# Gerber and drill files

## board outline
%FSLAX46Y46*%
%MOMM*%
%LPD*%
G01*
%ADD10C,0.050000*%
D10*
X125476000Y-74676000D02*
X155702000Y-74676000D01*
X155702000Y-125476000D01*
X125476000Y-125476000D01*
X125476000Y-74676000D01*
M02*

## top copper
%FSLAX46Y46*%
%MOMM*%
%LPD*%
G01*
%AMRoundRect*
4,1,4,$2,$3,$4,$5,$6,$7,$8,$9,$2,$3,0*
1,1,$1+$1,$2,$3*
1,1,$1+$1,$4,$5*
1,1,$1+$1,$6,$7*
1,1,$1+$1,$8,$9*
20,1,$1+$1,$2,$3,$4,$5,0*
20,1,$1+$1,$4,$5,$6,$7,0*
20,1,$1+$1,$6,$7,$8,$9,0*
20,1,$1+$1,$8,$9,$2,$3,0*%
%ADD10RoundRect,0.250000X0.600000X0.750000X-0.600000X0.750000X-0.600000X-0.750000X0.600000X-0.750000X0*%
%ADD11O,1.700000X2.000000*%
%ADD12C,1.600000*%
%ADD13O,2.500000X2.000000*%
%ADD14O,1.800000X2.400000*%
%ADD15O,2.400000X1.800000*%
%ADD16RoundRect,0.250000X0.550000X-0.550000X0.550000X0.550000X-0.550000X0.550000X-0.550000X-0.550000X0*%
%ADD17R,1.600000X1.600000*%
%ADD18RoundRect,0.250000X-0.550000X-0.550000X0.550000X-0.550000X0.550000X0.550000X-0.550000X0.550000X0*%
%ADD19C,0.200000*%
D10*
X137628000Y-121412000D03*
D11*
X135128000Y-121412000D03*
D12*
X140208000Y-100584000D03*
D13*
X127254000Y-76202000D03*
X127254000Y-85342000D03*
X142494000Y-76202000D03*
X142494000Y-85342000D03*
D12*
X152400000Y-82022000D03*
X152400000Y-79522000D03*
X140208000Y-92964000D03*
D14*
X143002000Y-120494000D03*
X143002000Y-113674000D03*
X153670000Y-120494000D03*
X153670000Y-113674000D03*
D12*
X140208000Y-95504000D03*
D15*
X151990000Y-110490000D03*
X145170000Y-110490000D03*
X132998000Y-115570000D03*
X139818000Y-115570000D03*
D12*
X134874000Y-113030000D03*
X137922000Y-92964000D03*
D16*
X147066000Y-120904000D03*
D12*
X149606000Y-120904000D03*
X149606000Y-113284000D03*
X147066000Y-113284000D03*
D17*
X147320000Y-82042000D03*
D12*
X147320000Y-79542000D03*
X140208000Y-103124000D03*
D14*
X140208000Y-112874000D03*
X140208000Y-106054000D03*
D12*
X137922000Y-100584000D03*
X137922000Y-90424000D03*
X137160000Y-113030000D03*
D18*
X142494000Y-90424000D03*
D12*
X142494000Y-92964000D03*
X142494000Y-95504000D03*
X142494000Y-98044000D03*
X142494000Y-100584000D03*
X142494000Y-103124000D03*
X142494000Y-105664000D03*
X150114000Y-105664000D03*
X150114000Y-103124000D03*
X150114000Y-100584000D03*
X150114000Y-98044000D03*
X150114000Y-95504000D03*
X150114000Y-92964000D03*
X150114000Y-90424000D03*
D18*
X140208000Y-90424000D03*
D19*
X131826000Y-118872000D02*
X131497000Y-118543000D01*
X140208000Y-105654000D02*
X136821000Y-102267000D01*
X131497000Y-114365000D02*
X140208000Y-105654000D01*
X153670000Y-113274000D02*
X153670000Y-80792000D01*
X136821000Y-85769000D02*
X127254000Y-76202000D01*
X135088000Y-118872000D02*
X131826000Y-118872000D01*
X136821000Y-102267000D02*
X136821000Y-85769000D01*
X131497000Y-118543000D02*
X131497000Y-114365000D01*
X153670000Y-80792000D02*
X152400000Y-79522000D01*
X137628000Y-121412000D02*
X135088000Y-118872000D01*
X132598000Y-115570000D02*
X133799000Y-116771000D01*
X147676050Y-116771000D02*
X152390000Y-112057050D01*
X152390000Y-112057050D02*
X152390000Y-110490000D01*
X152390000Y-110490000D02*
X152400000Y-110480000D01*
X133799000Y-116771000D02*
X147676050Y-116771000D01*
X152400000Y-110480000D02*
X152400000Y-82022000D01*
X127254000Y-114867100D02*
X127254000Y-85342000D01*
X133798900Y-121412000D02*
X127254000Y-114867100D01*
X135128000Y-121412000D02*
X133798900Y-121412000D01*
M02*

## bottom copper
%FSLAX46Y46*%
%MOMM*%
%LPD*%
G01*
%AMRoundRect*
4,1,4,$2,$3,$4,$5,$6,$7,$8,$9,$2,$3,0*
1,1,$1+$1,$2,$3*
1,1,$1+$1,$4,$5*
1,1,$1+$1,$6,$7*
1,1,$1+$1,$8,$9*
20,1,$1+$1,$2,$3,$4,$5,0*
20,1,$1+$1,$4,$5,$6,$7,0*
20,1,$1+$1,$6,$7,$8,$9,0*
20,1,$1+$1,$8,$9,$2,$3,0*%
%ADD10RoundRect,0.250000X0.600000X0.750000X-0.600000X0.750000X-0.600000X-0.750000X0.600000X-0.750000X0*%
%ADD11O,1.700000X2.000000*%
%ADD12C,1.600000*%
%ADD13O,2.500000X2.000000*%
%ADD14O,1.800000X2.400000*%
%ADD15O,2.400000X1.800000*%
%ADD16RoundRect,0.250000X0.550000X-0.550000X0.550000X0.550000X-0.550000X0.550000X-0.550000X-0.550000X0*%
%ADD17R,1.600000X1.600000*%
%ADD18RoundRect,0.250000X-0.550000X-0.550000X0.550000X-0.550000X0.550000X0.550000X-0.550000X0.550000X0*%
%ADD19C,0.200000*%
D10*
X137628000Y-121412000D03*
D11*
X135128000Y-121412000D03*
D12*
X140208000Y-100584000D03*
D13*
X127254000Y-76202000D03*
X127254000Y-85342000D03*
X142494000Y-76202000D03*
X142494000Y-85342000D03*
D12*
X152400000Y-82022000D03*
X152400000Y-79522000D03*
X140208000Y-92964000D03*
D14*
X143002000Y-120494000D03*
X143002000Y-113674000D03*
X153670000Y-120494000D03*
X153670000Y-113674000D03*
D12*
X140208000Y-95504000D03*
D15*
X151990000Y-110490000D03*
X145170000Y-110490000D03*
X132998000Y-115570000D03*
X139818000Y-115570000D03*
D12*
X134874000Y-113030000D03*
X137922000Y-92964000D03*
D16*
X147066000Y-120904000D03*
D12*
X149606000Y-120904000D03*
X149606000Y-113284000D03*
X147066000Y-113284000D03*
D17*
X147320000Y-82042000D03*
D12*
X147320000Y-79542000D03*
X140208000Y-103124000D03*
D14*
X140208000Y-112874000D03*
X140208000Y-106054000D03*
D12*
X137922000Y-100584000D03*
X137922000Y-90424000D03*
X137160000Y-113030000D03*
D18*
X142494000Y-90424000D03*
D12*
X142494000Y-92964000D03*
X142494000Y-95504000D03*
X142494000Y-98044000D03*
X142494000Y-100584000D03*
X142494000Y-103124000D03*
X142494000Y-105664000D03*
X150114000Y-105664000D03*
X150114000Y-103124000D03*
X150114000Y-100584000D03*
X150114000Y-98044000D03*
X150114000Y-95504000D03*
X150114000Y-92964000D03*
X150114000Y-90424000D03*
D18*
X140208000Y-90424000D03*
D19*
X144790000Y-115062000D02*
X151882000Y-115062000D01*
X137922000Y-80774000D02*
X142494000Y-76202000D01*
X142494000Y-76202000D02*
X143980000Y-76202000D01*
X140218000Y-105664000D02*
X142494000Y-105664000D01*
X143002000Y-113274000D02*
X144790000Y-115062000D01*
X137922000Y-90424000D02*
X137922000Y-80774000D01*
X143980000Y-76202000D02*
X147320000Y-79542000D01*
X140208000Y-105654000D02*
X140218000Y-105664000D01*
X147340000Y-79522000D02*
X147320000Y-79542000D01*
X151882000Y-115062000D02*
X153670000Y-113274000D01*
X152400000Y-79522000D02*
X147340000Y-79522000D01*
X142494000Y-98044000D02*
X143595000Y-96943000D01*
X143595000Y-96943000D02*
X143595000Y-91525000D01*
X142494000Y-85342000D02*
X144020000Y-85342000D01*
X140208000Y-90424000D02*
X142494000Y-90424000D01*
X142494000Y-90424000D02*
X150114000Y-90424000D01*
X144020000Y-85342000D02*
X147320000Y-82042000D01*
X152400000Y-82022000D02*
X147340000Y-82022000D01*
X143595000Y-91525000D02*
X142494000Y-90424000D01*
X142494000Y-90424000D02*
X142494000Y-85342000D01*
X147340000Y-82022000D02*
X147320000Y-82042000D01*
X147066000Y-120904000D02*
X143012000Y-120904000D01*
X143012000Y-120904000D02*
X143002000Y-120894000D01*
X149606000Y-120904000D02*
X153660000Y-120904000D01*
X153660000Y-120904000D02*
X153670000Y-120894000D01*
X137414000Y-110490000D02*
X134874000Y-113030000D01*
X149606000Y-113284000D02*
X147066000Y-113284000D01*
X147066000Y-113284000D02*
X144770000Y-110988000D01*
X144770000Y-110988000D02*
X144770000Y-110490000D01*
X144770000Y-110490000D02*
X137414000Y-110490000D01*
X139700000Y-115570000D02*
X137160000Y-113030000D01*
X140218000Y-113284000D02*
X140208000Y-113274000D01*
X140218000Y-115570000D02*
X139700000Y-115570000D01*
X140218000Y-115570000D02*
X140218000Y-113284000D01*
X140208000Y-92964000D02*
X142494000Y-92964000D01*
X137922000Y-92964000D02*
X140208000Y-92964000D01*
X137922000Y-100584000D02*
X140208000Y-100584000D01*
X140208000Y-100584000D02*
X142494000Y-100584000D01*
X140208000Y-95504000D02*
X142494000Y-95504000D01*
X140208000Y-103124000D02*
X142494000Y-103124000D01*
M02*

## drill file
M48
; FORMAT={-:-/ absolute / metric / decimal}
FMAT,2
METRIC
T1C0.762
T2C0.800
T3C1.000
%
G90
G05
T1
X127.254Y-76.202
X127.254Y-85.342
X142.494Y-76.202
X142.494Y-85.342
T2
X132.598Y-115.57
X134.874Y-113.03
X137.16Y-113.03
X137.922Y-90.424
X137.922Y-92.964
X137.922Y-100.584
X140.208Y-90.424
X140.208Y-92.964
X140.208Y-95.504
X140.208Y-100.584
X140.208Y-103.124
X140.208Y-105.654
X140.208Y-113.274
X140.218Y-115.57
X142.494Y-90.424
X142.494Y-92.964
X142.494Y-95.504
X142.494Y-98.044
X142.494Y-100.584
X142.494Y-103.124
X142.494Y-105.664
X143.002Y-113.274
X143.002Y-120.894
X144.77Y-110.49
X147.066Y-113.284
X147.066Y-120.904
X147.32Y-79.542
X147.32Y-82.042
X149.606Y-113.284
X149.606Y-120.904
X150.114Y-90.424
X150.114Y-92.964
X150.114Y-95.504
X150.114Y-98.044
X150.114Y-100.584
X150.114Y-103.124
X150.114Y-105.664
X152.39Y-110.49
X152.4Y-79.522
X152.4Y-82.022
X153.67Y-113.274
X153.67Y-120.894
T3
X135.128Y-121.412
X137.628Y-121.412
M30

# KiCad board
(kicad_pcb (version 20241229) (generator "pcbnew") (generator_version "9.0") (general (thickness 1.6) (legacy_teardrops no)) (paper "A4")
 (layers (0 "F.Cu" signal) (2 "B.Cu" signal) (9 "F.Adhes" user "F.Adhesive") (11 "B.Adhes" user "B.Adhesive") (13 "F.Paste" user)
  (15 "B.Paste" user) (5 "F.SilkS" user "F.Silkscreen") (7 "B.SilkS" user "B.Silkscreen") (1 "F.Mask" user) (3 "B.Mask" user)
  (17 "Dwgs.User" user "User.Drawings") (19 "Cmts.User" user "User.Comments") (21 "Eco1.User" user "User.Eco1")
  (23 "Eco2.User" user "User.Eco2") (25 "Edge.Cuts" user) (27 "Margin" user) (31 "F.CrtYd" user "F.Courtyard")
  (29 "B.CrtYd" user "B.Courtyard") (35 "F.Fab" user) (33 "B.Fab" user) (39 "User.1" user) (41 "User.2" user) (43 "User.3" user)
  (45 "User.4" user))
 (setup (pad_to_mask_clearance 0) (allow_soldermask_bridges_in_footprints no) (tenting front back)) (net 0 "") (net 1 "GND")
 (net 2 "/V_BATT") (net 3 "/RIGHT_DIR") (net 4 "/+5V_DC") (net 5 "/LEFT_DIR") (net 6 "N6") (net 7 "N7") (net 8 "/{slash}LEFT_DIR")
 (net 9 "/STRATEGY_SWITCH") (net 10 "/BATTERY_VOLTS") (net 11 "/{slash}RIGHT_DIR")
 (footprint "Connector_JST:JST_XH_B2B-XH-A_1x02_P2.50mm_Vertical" (layer "F.Cu") (at 137.628 121.412 180)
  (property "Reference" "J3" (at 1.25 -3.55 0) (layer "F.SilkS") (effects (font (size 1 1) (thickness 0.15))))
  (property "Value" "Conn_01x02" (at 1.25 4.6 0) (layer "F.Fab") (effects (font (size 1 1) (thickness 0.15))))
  (pad "1" thru_hole roundrect (at 0 0 180) (size 1.7 2) (drill 1) (layers "*.Cu" "*.Mask") (remove_unused_layers no)
   (roundrect_rratio 0.147059) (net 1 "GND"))
  (pad "2" thru_hole oval (at 2.5 0 180) (size 1.7 2) (drill 1) (layers "*.Cu" "*.Mask") (remove_unused_layers no) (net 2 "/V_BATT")))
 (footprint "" (layer "F.Cu") (at 140.208 100.584)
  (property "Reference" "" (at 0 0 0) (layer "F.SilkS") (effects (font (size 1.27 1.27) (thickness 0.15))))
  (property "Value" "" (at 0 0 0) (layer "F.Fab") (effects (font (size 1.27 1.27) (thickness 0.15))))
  (pad "5" thru_hole circle (at 0 0) (size 1.6 1.6) (drill 0.8) (layers "*.Cu" "*.Mask") (remove_unused_layers no) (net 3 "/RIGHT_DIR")))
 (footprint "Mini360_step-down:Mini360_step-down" (layer "F.Cu") (at 134.874 80.772)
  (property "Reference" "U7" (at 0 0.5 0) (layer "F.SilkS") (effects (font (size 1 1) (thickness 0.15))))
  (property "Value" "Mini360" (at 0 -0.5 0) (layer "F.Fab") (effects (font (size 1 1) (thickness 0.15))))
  (pad "1" thru_hole oval (at -7.62 -4.57) (size 2.5 2) (drill 0.762) (layers "*.Cu" "*.Mask") (remove_unused_layers no) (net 1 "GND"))
  (pad "2" thru_hole oval (at -7.62 4.57) (size 2.5 2) (drill 0.762) (layers "*.Cu" "*.Mask") (remove_unused_layers no) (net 2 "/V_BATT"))
  (pad "3" thru_hole oval (at 7.62 -4.57) (size 2.5 2) (drill 0.762) (layers "*.Cu" "*.Mask") (remove_unused_layers no) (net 1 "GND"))
  (pad "4" thru_hole oval (at 7.62 4.57) (size 2.5 2) (drill 0.762) (layers "*.Cu" "*.Mask") (remove_unused_layers no) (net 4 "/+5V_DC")))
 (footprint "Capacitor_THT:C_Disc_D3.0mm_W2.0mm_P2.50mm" (layer "F.Cu") (at 152.4 82.022 90)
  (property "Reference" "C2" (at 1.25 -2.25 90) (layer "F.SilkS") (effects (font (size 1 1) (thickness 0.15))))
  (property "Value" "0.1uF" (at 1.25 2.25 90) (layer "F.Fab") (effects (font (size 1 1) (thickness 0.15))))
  (pad "1" thru_hole circle (at 0 0 90) (size 1.6 1.6) (drill 0.8) (layers "*.Cu" "*.Mask") (remove_unused_layers no) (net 4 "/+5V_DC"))
  (pad "2" thru_hole circle (at 2.5 0 90) (size 1.6 1.6) (drill 0.8) (layers "*.Cu" "*.Mask") (remove_unused_layers no) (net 1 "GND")))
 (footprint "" (layer "F.Cu") (at 140.208 92.964)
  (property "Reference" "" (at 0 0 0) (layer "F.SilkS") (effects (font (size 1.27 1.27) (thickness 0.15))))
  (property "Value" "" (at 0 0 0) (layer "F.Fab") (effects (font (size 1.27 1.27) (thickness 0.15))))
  (pad "2" thru_hole circle (at 0 0) (size 1.6 1.6) (drill 0.8) (layers "*.Cu" "*.Mask") (remove_unused_layers no) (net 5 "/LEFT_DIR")))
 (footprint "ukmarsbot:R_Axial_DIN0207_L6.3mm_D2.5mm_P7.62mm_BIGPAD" (layer "F.Cu") (at 143.002 120.894 90)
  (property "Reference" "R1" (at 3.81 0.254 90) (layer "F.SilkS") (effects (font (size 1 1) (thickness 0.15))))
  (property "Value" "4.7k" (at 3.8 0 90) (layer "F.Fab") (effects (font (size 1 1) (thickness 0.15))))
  (pad "1" thru_hole oval (at 0 0 90) (size 2.4 1.8) (drill 0.8 (offset 0.4 0)) (layers "*.Cu" "*.Mask") (remove_unused_layers no)
   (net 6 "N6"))
  (pad "2" thru_hole oval (at 7.62 0 90) (size 2.4 1.8) (drill 0.8 (offset -0.4 0)) (layers "*.Cu" "*.Mask") (remove_unused_layers no)
   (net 1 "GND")))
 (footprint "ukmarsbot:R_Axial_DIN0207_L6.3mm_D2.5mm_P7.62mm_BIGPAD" (layer "F.Cu") (at 153.67 120.894 90)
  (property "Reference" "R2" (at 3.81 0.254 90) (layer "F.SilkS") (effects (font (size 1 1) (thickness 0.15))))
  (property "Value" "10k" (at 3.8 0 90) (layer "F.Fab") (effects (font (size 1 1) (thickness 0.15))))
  (pad "1" thru_hole oval (at 0 0 90) (size 2.4 1.8) (drill 0.8 (offset 0.4 0)) (layers "*.Cu" "*.Mask") (remove_unused_layers no)
   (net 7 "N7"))
  (pad "2" thru_hole oval (at 7.62 0 90) (size 2.4 1.8) (drill 0.8 (offset -0.4 0)) (layers "*.Cu" "*.Mask") (remove_unused_layers no)
   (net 1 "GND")))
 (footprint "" (layer "F.Cu") (at 140.208 95.504)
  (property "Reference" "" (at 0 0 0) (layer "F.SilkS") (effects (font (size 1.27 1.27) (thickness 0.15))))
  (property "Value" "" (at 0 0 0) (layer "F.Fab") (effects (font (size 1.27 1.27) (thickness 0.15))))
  (pad "3" thru_hole circle (at 0 0) (size 1.6 1.6) (drill 0.8) (layers "*.Cu" "*.Mask") (remove_unused_layers no)
   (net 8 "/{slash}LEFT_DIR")))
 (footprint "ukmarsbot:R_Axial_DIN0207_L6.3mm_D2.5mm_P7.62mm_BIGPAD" (layer "F.Cu") (at 152.39 110.49 180)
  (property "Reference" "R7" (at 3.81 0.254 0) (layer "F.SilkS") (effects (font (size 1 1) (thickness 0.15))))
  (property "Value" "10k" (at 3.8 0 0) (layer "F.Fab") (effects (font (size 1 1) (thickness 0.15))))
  (pad "1" thru_hole oval (at 0 0 180) (size 2.4 1.8) (drill 0.8 (offset 0.4 0)) (layers "*.Cu" "*.Mask") (remove_unused_layers no)
   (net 4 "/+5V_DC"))
  (pad "2" thru_hole oval (at 7.62 0 180) (size 2.4 1.8) (drill 0.8 (offset -0.4 0)) (layers "*.Cu" "*.Mask") (remove_unused_layers no)
   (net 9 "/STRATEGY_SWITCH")))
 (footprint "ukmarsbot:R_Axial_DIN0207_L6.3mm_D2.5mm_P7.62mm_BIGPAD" (layer "F.Cu") (at 132.598 115.57)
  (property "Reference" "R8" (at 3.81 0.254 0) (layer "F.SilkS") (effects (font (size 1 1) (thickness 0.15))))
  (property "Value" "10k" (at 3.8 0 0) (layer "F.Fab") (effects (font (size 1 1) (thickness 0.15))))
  (pad "1" thru_hole oval (at 0 0) (size 2.4 1.8) (drill 0.8 (offset 0.4 0)) (layers "*.Cu" "*.Mask") (remove_unused_layers no)
   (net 4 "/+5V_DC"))
  (pad "2" thru_hole oval (at 7.62 0) (size 2.4 1.8) (drill 0.8 (offset -0.4 0)) (layers "*.Cu" "*.Mask") (remove_unused_layers no)
   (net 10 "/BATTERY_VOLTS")))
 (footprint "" (layer "F.Cu") (at 134.874 113.03)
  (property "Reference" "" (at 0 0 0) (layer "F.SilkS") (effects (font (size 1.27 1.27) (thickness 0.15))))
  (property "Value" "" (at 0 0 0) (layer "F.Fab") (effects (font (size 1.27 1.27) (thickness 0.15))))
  (pad "5" thru_hole circle (at 0 0) (size 1.6 1.6) (drill 0.8) (layers "*.Cu" "*.Mask") (remove_unused_layers no)
   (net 9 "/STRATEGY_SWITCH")))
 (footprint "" (layer "F.Cu") (at 137.922 92.964)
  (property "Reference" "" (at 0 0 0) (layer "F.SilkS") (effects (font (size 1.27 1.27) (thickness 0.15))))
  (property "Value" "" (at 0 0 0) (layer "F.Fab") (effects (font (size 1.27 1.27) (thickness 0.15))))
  (pad "2" thru_hole circle (at 0 0) (size 1.6 1.6) (drill 0.8) (layers "*.Cu" "*.Mask") (remove_unused_layers no) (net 5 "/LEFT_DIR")))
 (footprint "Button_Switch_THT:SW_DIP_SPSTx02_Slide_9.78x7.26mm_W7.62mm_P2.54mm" (layer "F.Cu") (at 147.066 120.904 90)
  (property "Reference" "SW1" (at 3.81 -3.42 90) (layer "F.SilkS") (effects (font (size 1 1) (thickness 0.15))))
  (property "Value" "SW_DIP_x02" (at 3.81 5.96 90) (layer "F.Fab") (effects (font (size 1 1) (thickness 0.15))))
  (pad "1" thru_hole roundrect (at 0 0 90) (size 1.6 1.6) (drill 0.8) (layers "*.Cu" "*.Mask") (remove_unused_layers no)
   (roundrect_rratio 0.15625) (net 6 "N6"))
  (pad "2" thru_hole circle (at 0 2.54 90) (size 1.6 1.6) (drill 0.8) (layers "*.Cu" "*.Mask") (remove_unused_layers no) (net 7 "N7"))
  (pad "3" thru_hole circle (at 7.62 2.54 90) (size 1.6 1.6) (drill 0.8) (layers "*.Cu" "*.Mask") (remove_unused_layers no)
   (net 9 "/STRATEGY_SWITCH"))
  (pad "4" thru_hole circle (at 7.62 0 90) (size 1.6 1.6) (drill 0.8) (layers "*.Cu" "*.Mask") (remove_unused_layers no)
   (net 9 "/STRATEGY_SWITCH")))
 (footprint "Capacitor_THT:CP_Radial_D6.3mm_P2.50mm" (layer "F.Cu") (at 147.32 82.042 90)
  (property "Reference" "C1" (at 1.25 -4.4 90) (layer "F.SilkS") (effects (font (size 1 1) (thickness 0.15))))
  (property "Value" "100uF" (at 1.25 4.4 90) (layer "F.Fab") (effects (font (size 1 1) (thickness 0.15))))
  (pad "1" thru_hole rect (at 0 0 90) (size 1.6 1.6) (drill 0.8) (layers "*.Cu" "*.Mask") (remove_unused_layers no) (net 4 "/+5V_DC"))
  (pad "2" thru_hole circle (at 2.5 0 90) (size 1.6 1.6) (drill 0.8) (layers "*.Cu" "*.Mask") (remove_unused_layers no) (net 1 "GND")))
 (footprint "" (layer "F.Cu") (at 140.208 103.124)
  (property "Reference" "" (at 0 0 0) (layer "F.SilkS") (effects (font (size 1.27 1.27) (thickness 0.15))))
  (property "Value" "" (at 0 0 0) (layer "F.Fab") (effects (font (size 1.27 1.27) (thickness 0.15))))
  (pad "6" thru_hole circle (at 0 0) (size 1.6 1.6) (drill 0.8) (layers "*.Cu" "*.Mask") (remove_unused_layers no)
   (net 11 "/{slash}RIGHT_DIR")))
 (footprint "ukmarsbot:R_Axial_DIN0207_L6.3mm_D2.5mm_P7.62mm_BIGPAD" (layer "F.Cu") (at 140.208 113.274 90)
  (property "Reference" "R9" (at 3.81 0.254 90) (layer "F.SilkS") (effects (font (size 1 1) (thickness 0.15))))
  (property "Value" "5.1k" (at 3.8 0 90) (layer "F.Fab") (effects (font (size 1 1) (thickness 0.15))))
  (pad "1" thru_hole oval (at 0 0 90) (size 2.4 1.8) (drill 0.8 (offset 0.4 0)) (layers "*.Cu" "*.Mask") (remove_unused_layers no)
   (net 10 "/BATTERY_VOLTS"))
  (pad "2" thru_hole oval (at 7.62 0 90) (size 2.4 1.8) (drill 0.8 (offset -0.4 0)) (layers "*.Cu" "*.Mask") (remove_unused_layers no)
   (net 1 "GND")))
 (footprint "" (layer "F.Cu") (at 137.922 100.584)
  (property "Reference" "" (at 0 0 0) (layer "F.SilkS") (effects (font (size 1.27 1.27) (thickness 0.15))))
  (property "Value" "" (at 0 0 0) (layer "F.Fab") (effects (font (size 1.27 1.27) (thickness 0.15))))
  (pad "5" thru_hole circle (at 0 0) (size 1.6 1.6) (drill 0.8) (layers "*.Cu" "*.Mask") (remove_unused_layers no) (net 3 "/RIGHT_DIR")))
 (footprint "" (layer "F.Cu") (at 137.922 90.424)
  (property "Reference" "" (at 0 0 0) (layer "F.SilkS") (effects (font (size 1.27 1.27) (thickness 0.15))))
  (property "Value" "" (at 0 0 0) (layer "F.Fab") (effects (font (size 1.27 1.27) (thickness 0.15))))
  (pad "2" thru_hole circle (at 0 0 90) (size 1.6 1.6) (drill 0.8) (layers "*.Cu" "*.Mask") (remove_unused_layers no) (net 1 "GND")))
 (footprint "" (layer "F.Cu") (at 137.16 113.03)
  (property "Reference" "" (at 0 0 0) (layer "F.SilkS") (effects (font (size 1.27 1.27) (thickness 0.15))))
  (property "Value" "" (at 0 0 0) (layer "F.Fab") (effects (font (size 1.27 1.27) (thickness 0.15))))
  (pad "5" thru_hole circle (at 0 0) (size 1.6 1.6) (drill 0.8) (layers "*.Cu" "*.Mask") (remove_unused_layers no) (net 10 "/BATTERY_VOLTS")))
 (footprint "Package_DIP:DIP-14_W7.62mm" (layer "F.Cu") (at 142.494 90.424)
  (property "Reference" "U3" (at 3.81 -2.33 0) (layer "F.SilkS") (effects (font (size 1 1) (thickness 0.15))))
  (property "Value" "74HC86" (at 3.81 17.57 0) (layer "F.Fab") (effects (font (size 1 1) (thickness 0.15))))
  (pad "1" thru_hole roundrect (at 0 0) (size 1.6 1.6) (drill 0.8) (layers "*.Cu" "*.Mask") (remove_unused_layers no)
   (roundrect_rratio 0.15625) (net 4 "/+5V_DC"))
  (pad "2" thru_hole circle (at 0 2.54) (size 1.6 1.6) (drill 0.8) (layers "*.Cu" "*.Mask") (remove_unused_layers no) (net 5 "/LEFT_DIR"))
  (pad "3" thru_hole circle (at 0 5.08) (size 1.6 1.6) (drill 0.8) (layers "*.Cu" "*.Mask") (remove_unused_layers no)
   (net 8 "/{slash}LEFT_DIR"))
  (pad "4" thru_hole circle (at 0 7.62) (size 1.6 1.6) (drill 0.8) (layers "*.Cu" "*.Mask") (remove_unused_layers no) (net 4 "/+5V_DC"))
  (pad "5" thru_hole circle (at 0 10.16) (size 1.6 1.6) (drill 0.8) (layers "*.Cu" "*.Mask") (remove_unused_layers no) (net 3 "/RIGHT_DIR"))
  (pad "6" thru_hole circle (at 0 12.7) (size 1.6 1.6) (drill 0.8) (layers "*.Cu" "*.Mask") (remove_unused_layers no)
   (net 11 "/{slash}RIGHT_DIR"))
  (pad "7" thru_hole circle (at 0 15.24) (size 1.6 1.6) (drill 0.8) (layers "*.Cu" "*.Mask") (remove_unused_layers no) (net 1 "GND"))
  (pad "8" thru_hole circle (at 7.62 15.24) (size 1.6 1.6) (drill 0.8) (layers "*.Cu" "*.Mask") (remove_unused_layers no))
  (pad "9" thru_hole circle (at 7.62 12.7) (size 1.6 1.6) (drill 0.8) (layers "*.Cu" "*.Mask") (remove_unused_layers no))
  (pad "10" thru_hole circle (at 7.62 10.16) (size 1.6 1.6) (drill 0.8) (layers "*.Cu" "*.Mask") (remove_unused_layers no))
  (pad "11" thru_hole circle (at 7.62 7.62) (size 1.6 1.6) (drill 0.8) (layers "*.Cu" "*.Mask") (remove_unused_layers no))
  (pad "12" thru_hole circle (at 7.62 5.08) (size 1.6 1.6) (drill 0.8) (layers "*.Cu" "*.Mask") (remove_unused_layers no))
  (pad "13" thru_hole circle (at 7.62 2.54) (size 1.6 1.6) (drill 0.8) (layers "*.Cu" "*.Mask") (remove_unused_layers no))
  (pad "14" thru_hole circle (at 7.62 0) (size 1.6 1.6) (drill 0.8) (layers "*.Cu" "*.Mask") (remove_unused_layers no)))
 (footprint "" (layer "F.Cu") (at 140.208 90.424)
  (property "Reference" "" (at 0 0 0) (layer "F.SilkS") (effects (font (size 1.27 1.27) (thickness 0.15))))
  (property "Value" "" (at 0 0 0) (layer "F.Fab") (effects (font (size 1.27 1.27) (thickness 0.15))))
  (pad "1" thru_hole roundrect (at 0 0) (size 1.6 1.6) (drill 0.8) (layers "*.Cu" "*.Mask") (remove_unused_layers no)
   (roundrect_rratio 0.15625) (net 4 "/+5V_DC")))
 (gr_rect (start 125.476 74.676) (end 155.702 125.476) (stroke (width 0.05) (type default)) (fill no) (layer "Edge.Cuts"))
 (segment (start 131.826 118.872) (end 131.497 118.543) (width 0.2) (layer "F.Cu") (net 1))
 (segment (start 140.208 105.654) (end 136.821 102.267) (width 0.2) (layer "F.Cu") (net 1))
 (segment (start 131.497 114.365) (end 140.208 105.654) (width 0.2) (layer "F.Cu") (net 1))
 (segment (start 153.67 113.274) (end 153.67 80.792) (width 0.2) (layer "F.Cu") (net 1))
 (segment (start 136.821 85.769) (end 127.254 76.202) (width 0.2) (layer "F.Cu") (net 1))
 (segment (start 135.088 118.872) (end 131.826 118.872) (width 0.2) (layer "F.Cu") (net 1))
 (segment (start 136.821 102.267) (end 136.821 85.769) (width 0.2) (layer "F.Cu") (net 1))
 (segment (start 131.497 118.543) (end 131.497 114.365) (width 0.2) (layer "F.Cu") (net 1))
 (segment (start 153.67 80.792) (end 152.4 79.522) (width 0.2) (layer "F.Cu") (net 1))
 (segment (start 137.628 121.412) (end 135.088 118.872) (width 0.2) (layer "F.Cu") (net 1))
 (segment (start 144.79 115.062) (end 151.882 115.062) (width 0.2) (layer "B.Cu") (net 1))
 (segment (start 137.922 80.774) (end 142.494 76.202) (width 0.2) (layer "B.Cu") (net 1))
 (segment (start 142.494 76.202) (end 143.98 76.202) (width 0.2) (layer "B.Cu") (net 1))
 (segment (start 140.218 105.664) (end 142.494 105.664) (width 0.2) (layer "B.Cu") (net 1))
 (segment (start 143.002 113.274) (end 144.79 115.062) (width 0.2) (layer "B.Cu") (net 1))
 (segment (start 137.922 90.424) (end 137.922 80.774) (width 0.2) (layer "B.Cu") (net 1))
 (segment (start 143.98 76.202) (end 147.32 79.542) (width 0.2) (layer "B.Cu") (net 1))
 (segment (start 140.208 105.654) (end 140.218 105.664) (width 0.2) (layer "B.Cu") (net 1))
 (segment (start 147.34 79.522) (end 147.32 79.542) (width 0.2) (layer "B.Cu") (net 1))
 (segment (start 151.882 115.062) (end 153.67 113.274) (width 0.2) (layer "B.Cu") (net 1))
 (segment (start 152.4 79.522) (end 147.34 79.522) (width 0.2) (layer "B.Cu") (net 1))
 (segment (start 132.598 115.57) (end 133.799 116.771) (width 0.2) (layer "F.Cu") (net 4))
 (segment (start 147.67605 116.771) (end 152.39 112.05705) (width 0.2) (layer "F.Cu") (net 4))
 (segment (start 152.39 112.05705) (end 152.39 110.49) (width 0.2) (layer "F.Cu") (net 4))
 (segment (start 152.39 110.49) (end 152.4 110.48) (width 0.2) (layer "F.Cu") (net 4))
 (segment (start 133.799 116.771) (end 147.67605 116.771) (width 0.2) (layer "F.Cu") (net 4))
 (segment (start 152.4 110.48) (end 152.4 82.022) (width 0.2) (layer "F.Cu") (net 4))
 (segment (start 142.494 98.044) (end 143.595 96.943) (width 0.2) (layer "B.Cu") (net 4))
 (segment (start 143.595 96.943) (end 143.595 91.525) (width 0.2) (layer "B.Cu") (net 4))
 (segment (start 142.494 85.342) (end 144.02 85.342) (width 0.2) (layer "B.Cu") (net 4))
 (segment (start 140.208 90.424) (end 142.494 90.424) (width 0.2) (layer "B.Cu") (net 4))
 (segment (start 142.494 90.424) (end 150.114 90.424) (width 0.2) (layer "B.Cu") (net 4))
 (segment (start 144.02 85.342) (end 147.32 82.042) (width 0.2) (layer "B.Cu") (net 4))
 (segment (start 152.4 82.022) (end 147.34 82.022) (width 0.2) (layer "B.Cu") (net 4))
 (segment (start 143.595 91.525) (end 142.494 90.424) (width 0.2) (layer "B.Cu") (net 4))
 (segment (start 142.494 90.424) (end 142.494 85.342) (width 0.2) (layer "B.Cu") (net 4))
 (segment (start 147.34 82.022) (end 147.32 82.042) (width 0.2) (layer "B.Cu") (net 4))
 (segment (start 127.254 114.8671) (end 127.254 85.342) (width 0.2) (layer "F.Cu") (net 2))
 (segment (start 133.7989 121.412) (end 127.254 114.8671) (width 0.2) (layer "F.Cu") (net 2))
 (segment (start 135.128 121.412) (end 133.7989 121.412) (width 0.2) (layer "F.Cu") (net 2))
 (segment (start 147.066 120.904) (end 143.012 120.904) (width 0.2) (layer "B.Cu") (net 6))
 (segment (start 143.012 120.904) (end 143.002 120.894) (width 0.2) (layer "B.Cu") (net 6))
 (segment (start 149.606 120.904) (end 153.66 120.904) (width 0.2) (layer "B.Cu") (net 7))
 (segment (start 153.66 120.904) (end 153.67 120.894) (width 0.2) (layer "B.Cu") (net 7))
 (segment (start 137.414 110.49) (end 134.874 113.03) (width 0.2) (layer "B.Cu") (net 9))
 (segment (start 149.606 113.284) (end 147.066 113.284) (width 0.2) (layer "B.Cu") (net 9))
 (segment (start 147.066 113.284) (end 144.77 110.988) (width 0.2) (layer "B.Cu") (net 9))
 (segment (start 144.77 110.988) (end 144.77 110.49) (width 0.2) (layer "B.Cu") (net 9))
 (segment (start 144.77 110.49) (end 137.414 110.49) (width 0.2) (layer "B.Cu") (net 9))
 (segment (start 139.7 115.57) (end 137.16 113.03) (width 0.2) (layer "B.Cu") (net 10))
 (segment (start 140.218 113.284) (end 140.208 113.274) (width 0.2) (layer "B.Cu") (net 10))
 (segment (start 140.218 115.57) (end 139.7 115.57) (width 0.2) (layer "B.Cu") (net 10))
 (segment (start 140.218 115.57) (end 140.218 113.284) (width 0.2) (layer "B.Cu") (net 10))
 (segment (start 140.208 92.964) (end 142.494 92.964) (width 0.2) (layer "B.Cu") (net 5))
 (segment (start 137.922 92.964) (end 140.208 92.964) (width 0.2) (layer "B.Cu") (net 5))
 (segment (start 137.922 100.584) (end 140.208 100.584) (width 0.2) (layer "B.Cu") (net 3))
 (segment (start 140.208 100.584) (end 142.494 100.584) (width 0.2) (layer "B.Cu") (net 3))
 (segment (start 140.208 95.504) (end 142.494 95.504) (width 0.2) (layer "B.Cu") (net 8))
 (segment (start 140.208 103.124) (end 142.494 103.124) (width 0.2) (layer "B.Cu") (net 11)))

